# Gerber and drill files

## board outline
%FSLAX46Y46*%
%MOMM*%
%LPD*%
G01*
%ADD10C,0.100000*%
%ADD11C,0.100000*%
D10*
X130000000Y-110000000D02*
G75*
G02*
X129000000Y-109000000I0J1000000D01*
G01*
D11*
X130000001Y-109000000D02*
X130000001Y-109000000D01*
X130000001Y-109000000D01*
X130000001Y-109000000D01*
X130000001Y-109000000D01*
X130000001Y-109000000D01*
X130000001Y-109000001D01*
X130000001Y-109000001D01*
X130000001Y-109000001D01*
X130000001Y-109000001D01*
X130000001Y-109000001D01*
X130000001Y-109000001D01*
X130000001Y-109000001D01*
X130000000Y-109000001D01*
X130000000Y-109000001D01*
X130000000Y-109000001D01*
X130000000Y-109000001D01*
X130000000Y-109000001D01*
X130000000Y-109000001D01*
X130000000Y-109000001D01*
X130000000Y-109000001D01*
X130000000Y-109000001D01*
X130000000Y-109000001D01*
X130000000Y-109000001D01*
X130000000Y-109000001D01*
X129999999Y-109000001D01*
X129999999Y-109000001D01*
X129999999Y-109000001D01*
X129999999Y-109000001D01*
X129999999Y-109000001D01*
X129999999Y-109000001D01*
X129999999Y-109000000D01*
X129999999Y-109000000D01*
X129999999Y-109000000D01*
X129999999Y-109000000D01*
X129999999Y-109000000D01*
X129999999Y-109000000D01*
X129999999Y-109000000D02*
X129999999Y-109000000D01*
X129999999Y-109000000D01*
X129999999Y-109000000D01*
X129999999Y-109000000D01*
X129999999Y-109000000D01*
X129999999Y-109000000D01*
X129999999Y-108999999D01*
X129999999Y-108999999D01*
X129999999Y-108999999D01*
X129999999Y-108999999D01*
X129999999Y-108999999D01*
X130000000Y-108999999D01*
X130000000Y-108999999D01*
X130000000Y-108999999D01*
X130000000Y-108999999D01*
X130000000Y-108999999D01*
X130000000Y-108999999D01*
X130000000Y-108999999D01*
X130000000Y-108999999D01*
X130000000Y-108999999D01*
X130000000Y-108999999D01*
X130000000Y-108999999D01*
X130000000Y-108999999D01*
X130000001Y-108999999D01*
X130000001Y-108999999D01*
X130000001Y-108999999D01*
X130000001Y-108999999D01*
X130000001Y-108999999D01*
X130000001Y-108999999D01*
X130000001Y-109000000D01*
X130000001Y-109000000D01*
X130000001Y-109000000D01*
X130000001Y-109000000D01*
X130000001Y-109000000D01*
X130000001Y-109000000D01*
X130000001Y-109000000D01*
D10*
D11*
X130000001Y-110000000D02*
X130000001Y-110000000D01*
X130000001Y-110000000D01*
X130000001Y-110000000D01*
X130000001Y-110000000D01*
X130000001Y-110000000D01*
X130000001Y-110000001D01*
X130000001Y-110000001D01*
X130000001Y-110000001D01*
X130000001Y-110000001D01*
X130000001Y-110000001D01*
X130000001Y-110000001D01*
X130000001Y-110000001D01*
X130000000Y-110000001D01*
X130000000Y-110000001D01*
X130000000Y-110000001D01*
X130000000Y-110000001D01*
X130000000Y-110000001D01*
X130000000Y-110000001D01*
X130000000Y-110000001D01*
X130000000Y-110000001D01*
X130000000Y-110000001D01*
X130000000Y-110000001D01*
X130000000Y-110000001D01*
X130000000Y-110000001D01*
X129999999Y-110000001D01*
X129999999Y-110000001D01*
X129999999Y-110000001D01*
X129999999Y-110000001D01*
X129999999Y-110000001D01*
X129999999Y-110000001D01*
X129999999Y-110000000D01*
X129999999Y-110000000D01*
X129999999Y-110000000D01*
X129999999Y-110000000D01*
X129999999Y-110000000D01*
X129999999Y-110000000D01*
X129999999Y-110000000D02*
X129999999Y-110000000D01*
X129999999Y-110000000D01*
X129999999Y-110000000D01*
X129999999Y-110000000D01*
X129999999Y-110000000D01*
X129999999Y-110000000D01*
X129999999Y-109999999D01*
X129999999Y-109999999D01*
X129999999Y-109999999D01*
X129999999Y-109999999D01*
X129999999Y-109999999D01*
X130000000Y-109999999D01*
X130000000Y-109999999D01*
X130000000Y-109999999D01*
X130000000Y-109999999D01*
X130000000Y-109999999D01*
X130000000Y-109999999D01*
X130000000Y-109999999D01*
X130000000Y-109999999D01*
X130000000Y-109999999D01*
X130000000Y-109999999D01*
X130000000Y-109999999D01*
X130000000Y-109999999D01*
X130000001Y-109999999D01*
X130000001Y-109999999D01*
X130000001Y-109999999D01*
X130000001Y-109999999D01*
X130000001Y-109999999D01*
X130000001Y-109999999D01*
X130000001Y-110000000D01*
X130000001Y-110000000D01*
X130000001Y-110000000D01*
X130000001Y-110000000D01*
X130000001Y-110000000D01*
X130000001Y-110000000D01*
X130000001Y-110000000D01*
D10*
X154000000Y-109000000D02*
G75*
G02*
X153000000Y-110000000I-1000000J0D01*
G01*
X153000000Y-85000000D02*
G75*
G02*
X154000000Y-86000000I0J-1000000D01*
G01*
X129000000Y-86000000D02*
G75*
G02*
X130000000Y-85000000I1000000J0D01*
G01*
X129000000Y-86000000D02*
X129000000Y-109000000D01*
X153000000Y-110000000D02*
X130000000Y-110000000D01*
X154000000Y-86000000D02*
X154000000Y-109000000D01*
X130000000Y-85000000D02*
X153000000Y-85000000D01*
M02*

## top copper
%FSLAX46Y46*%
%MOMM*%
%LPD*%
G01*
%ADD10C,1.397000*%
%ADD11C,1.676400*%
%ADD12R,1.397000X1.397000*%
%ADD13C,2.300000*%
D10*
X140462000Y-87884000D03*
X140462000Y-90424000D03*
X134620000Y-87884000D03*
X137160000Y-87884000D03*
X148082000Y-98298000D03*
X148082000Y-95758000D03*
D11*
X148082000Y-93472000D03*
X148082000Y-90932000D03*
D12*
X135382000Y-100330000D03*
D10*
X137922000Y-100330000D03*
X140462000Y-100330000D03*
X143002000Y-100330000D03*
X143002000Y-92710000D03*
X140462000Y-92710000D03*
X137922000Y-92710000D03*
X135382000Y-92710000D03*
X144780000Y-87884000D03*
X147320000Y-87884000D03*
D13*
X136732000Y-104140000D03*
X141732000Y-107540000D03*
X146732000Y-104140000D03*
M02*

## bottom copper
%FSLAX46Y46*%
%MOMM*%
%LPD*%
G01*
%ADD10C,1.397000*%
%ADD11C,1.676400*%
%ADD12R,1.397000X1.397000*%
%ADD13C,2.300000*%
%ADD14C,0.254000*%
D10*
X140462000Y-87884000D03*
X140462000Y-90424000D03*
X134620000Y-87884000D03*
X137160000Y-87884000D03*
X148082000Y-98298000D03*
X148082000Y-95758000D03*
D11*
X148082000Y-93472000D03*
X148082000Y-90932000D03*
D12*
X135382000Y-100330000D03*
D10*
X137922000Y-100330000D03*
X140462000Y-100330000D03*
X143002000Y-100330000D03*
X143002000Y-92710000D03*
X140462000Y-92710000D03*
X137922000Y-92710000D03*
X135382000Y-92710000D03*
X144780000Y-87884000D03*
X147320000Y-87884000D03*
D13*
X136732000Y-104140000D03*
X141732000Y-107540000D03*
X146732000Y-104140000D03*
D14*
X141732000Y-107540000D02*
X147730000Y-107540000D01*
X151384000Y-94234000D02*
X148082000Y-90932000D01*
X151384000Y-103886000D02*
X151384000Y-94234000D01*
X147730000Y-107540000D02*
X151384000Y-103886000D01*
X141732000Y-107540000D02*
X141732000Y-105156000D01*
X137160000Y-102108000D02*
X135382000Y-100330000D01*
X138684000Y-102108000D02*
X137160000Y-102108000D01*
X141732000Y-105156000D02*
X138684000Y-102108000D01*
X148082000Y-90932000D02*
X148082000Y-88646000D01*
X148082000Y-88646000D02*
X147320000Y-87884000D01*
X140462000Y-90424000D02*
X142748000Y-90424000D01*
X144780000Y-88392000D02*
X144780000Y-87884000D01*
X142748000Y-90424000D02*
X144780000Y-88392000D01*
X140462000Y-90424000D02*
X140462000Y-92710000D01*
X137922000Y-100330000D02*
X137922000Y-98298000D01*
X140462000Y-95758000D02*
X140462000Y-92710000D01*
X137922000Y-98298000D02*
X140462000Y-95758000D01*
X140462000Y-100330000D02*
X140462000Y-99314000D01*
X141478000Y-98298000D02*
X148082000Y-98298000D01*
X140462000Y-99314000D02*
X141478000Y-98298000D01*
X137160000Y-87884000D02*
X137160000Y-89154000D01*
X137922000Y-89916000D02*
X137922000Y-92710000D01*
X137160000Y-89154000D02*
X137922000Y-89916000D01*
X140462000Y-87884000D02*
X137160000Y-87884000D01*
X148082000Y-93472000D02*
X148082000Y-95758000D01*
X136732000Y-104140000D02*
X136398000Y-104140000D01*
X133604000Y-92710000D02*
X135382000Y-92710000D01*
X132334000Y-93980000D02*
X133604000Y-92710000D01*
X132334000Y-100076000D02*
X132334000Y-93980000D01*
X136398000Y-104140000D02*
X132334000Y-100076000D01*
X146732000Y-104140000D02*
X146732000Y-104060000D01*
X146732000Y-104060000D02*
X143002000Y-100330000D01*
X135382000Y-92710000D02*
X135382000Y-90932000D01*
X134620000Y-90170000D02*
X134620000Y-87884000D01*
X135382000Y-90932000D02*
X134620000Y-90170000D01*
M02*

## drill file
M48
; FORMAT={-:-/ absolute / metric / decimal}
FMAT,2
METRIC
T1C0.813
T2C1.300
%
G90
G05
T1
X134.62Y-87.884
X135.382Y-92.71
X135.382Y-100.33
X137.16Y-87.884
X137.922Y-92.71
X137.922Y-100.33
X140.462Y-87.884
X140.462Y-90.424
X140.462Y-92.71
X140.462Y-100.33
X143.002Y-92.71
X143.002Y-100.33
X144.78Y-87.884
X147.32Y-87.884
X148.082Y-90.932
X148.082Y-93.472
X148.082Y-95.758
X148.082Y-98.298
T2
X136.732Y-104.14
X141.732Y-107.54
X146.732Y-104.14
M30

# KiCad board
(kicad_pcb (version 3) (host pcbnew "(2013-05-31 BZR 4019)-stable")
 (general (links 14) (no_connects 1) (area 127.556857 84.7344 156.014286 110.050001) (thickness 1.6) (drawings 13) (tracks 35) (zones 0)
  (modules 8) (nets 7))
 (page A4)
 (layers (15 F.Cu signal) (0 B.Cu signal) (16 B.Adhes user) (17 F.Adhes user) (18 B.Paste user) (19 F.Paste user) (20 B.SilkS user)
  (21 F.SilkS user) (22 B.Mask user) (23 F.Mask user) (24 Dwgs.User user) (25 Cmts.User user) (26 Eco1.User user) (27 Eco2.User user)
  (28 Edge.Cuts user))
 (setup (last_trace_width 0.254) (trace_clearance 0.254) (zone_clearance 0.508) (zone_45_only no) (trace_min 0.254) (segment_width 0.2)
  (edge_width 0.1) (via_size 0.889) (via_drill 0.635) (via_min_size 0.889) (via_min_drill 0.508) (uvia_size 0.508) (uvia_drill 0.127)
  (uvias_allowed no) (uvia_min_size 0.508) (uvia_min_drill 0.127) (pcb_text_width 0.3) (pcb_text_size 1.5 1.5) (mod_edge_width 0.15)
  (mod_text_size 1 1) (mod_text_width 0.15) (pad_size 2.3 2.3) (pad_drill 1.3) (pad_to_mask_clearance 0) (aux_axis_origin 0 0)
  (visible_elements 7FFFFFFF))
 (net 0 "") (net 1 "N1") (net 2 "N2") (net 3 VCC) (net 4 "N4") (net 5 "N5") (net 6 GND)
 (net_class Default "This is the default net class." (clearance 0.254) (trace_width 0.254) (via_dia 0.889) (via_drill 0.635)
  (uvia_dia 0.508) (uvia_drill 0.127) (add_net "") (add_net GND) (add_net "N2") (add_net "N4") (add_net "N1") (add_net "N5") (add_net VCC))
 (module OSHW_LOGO (layer B.Cu) (at 132.08 106.172 90)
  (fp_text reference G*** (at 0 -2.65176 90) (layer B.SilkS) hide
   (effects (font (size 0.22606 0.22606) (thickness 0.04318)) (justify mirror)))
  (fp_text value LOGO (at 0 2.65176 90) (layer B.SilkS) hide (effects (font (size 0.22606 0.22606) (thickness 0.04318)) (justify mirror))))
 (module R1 (layer F.Cu) (at 140.462 89.154 270) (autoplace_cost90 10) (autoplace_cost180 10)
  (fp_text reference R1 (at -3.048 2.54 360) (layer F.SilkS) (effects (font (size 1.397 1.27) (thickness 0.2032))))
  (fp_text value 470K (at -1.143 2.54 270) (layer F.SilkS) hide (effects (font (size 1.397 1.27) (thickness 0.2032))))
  (pad 1 thru_hole circle (at -1.27 0 270) (size 1.397 1.397) (drill 0.8128) (layers *.Cu *.Mask F.SilkS) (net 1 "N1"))
  (pad 2 thru_hole circle (at 1.27 0 270) (size 1.397 1.397) (drill 0.8128) (layers *.Cu *.Mask F.SilkS) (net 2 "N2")))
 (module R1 (layer F.Cu) (at 135.89 87.884) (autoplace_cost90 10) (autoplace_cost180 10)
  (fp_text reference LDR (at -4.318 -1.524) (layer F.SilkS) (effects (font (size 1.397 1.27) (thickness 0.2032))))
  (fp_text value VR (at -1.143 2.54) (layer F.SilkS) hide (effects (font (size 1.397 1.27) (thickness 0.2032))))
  (pad 1 thru_hole circle (at -1.27 0) (size 1.397 1.397) (drill 0.8128) (layers *.Cu *.Mask F.SilkS) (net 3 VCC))
  (pad 2 thru_hole circle (at 1.27 0) (size 1.397 1.397) (drill 0.8128) (layers *.Cu *.Mask F.SilkS) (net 1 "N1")))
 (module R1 (layer F.Cu) (at 148.082 97.028 90) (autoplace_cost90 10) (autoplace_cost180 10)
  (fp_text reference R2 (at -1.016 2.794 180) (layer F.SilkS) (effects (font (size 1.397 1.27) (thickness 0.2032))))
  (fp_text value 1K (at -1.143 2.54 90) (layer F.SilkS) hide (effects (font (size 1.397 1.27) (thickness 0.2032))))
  (pad 1 thru_hole circle (at -1.27 0 90) (size 1.397 1.397) (drill 0.8128) (layers *.Cu *.Mask F.SilkS) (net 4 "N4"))
  (pad 2 thru_hole circle (at 1.27 0 90) (size 1.397 1.397) (drill 0.8128) (layers *.Cu *.Mask F.SilkS) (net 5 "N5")))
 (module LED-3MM (layer F.Cu) (at 148.082 92.202 90)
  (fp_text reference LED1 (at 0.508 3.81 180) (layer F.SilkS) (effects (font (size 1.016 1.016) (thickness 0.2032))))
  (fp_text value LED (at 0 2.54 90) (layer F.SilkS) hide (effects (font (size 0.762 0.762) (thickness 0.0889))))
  (pad 1 thru_hole circle (at -1.27 0 90) (size 1.6764 1.6764) (drill 0.8128) (layers *.Cu *.Mask F.SilkS) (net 5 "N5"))
  (pad 2 thru_hole circle (at 1.27 0 90) (size 1.6764 1.6764) (drill 0.8128) (layers *.Cu *.Mask F.SilkS) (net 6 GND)))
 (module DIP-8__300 (layer F.Cu) (at 139.192 96.52)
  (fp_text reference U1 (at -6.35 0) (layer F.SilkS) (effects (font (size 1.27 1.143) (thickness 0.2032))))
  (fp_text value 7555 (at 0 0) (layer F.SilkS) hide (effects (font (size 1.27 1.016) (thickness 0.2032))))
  (pad 1 thru_hole rect (at -3.81 3.81) (size 1.397 1.397) (drill 0.8128) (layers *.Cu *.Mask F.SilkS) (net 6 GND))
  (pad 2 thru_hole circle (at -1.27 3.81) (size 1.397 1.397) (drill 0.8128) (layers *.Cu *.Mask F.SilkS) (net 2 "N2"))
  (pad 3 thru_hole circle (at 1.27 3.81) (size 1.397 1.397) (drill 0.8128) (layers *.Cu *.Mask F.SilkS) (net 4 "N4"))
  (pad 4 thru_hole circle (at 3.81 3.81) (size 1.397 1.397) (drill 0.8128) (layers *.Cu *.Mask F.SilkS) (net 3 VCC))
  (pad 5 thru_hole circle (at 3.81 -3.81) (size 1.397 1.397) (drill 0.8128) (layers *.Cu *.Mask F.SilkS))
  (pad 6 thru_hole circle (at 1.27 -3.81) (size 1.397 1.397) (drill 0.8128) (layers *.Cu *.Mask F.SilkS) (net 2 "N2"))
  (pad 7 thru_hole circle (at -1.27 -3.81) (size 1.397 1.397) (drill 0.8128) (layers *.Cu *.Mask F.SilkS) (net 1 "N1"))
  (pad 8 thru_hole circle (at -3.81 -3.81) (size 1.397 1.397) (drill 0.8128) (layers *.Cu *.Mask F.SilkS) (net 3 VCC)))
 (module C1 (layer F.Cu) (at 146.05 87.884)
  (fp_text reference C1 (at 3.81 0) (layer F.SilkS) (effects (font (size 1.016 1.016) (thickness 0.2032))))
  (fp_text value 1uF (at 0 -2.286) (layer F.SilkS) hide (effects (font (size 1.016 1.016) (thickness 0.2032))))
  (pad 1 thru_hole circle (at -1.27 0) (size 1.397 1.397) (drill 0.8128) (layers *.Cu *.Mask F.SilkS) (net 2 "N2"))
  (pad 2 thru_hole circle (at 1.27 0) (size 1.397 1.397) (drill 0.8128) (layers *.Cu *.Mask F.SilkS) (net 6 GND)))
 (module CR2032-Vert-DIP (layer F.Cu) (at 141.732 104.14 180)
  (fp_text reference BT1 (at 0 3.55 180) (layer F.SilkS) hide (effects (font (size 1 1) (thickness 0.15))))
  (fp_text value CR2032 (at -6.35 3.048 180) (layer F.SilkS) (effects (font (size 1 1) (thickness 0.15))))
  (pad 1 thru_hole circle (at 5 0 180) (size 2.3 2.3) (drill 1.3) (layers *.Cu *.Mask F.SilkS) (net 3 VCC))
  (pad 2 thru_hole circle (at 0 -3.4 180) (size 2.3 2.3) (drill 1.3) (layers *.Cu *.Mask F.SilkS) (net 6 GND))
  (pad 1 thru_hole circle (at -5 0 180) (size 2.3 2.3) (drill 1.3) (layers *.Cu *.Mask F.SilkS) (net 3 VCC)))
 (gr_arc (start 130 109) (end 130 110) (angle 90) (layer Edge.Cuts) (width 0.1))
 (gr_arc (start 130 109) (end 130 109) (angle 90) (layer Edge.Cuts) (width 0.1))
 (gr_arc (start 130 110) (end 130 110) (angle 90) (layer Edge.Cuts) (width 0.1))
 (gr_arc (start 153 109) (end 154 109) (angle 90) (layer Edge.Cuts) (width 0.1))
 (gr_arc (start 153 86) (end 153 85) (angle 90) (layer Edge.Cuts) (width 0.1))
 (gr_arc (start 130 86) (end 129 86) (angle 90) (layer Edge.Cuts) (width 0.1))
 (gr_line (start 129 86) (end 129 109) (angle 90) (layer Edge.Cuts) (width 0.1))
 (gr_line (start 153 110) (end 130 110) (angle 90) (layer Edge.Cuts) (width 0.1))
 (gr_line (start 154 86) (end 154 109) (angle 90) (layer Edge.Cuts) (width 0.1))
 (gr_line (start 130 85) (end 153 85) (angle 90) (layer Edge.Cuts) (width 0.1))
 (segment (start 141.732 107.54) (end 147.73 107.54) (width 0.254) (layer B.Cu) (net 6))
 (segment (start 151.384 94.234) (end 148.082 90.932) (width 0.254) (layer B.Cu) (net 6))
 (segment (start 151.384 103.886) (end 151.384 94.234) (width 0.254) (layer B.Cu) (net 6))
 (segment (start 147.73 107.54) (end 151.384 103.886) (width 0.254) (layer B.Cu) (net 6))
 (segment (start 141.732 107.54) (end 141.732 105.156) (width 0.254) (layer B.Cu) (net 6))
 (segment (start 137.16 102.108) (end 135.382 100.33) (width 0.254) (layer B.Cu) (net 6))
 (segment (start 138.684 102.108) (end 137.16 102.108) (width 0.254) (layer B.Cu) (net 6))
 (segment (start 141.732 105.156) (end 138.684 102.108) (width 0.254) (layer B.Cu) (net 6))
 (segment (start 148.082 90.932) (end 148.082 88.646) (width 0.254) (layer B.Cu) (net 6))
 (segment (start 148.082 88.646) (end 147.32 87.884) (width 0.254) (layer B.Cu) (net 6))
 (segment (start 140.462 90.424) (end 142.748 90.424) (width 0.254) (layer B.Cu) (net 2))
 (segment (start 144.78 88.392) (end 144.78 87.884) (width 0.254) (layer B.Cu) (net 2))
 (segment (start 142.748 90.424) (end 144.78 88.392) (width 0.254) (layer B.Cu) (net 2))
 (segment (start 140.462 90.424) (end 140.462 92.71) (width 0.254) (layer B.Cu) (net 2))
 (segment (start 137.922 100.33) (end 137.922 98.298) (width 0.254) (layer B.Cu) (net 2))
 (segment (start 140.462 95.758) (end 140.462 92.71) (width 0.254) (layer B.Cu) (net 2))
 (segment (start 137.922 98.298) (end 140.462 95.758) (width 0.254) (layer B.Cu) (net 2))
 (segment (start 140.462 100.33) (end 140.462 99.314) (width 0.254) (layer B.Cu) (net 4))
 (segment (start 141.478 98.298) (end 148.082 98.298) (width 0.254) (layer B.Cu) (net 4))
 (segment (start 140.462 99.314) (end 141.478 98.298) (width 0.254) (layer B.Cu) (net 4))
 (segment (start 137.16 87.884) (end 137.16 89.154) (width 0.254) (layer B.Cu) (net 1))
 (segment (start 137.922 89.916) (end 137.922 92.71) (width 0.254) (layer B.Cu) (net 1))
 (segment (start 137.16 89.154) (end 137.922 89.916) (width 0.254) (layer B.Cu) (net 1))
 (segment (start 140.462 87.884) (end 137.16 87.884) (width 0.254) (layer B.Cu) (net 1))
 (segment (start 148.082 93.472) (end 148.082 95.758) (width 0.254) (layer B.Cu) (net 5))
 (segment (start 136.732 104.14) (end 136.398 104.14) (width 0.254) (layer B.Cu) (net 3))
 (segment (start 133.604 92.71) (end 135.382 92.71) (width 0.254) (layer B.Cu) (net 3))
 (segment (start 132.334 93.98) (end 133.604 92.71) (width 0.254) (layer B.Cu) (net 3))
 (segment (start 132.334 100.076) (end 132.334 93.98) (width 0.254) (layer B.Cu) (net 3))
 (segment (start 136.398 104.14) (end 132.334 100.076) (width 0.254) (layer B.Cu) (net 3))
 (segment (start 146.732 104.14) (end 146.732 104.06) (width 0.254) (layer B.Cu) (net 3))
 (segment (start 146.732 104.06) (end 143.002 100.33) (width 0.254) (layer B.Cu) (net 3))
 (segment (start 135.382 92.71) (end 135.382 90.932) (width 0.254) (layer B.Cu) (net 3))
 (segment (start 134.62 90.17) (end 134.62 87.884) (width 0.254) (layer B.Cu) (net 3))
 (segment (start 135.382 90.932) (end 134.62 90.17) (width 0.254) (layer B.Cu) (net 3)))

